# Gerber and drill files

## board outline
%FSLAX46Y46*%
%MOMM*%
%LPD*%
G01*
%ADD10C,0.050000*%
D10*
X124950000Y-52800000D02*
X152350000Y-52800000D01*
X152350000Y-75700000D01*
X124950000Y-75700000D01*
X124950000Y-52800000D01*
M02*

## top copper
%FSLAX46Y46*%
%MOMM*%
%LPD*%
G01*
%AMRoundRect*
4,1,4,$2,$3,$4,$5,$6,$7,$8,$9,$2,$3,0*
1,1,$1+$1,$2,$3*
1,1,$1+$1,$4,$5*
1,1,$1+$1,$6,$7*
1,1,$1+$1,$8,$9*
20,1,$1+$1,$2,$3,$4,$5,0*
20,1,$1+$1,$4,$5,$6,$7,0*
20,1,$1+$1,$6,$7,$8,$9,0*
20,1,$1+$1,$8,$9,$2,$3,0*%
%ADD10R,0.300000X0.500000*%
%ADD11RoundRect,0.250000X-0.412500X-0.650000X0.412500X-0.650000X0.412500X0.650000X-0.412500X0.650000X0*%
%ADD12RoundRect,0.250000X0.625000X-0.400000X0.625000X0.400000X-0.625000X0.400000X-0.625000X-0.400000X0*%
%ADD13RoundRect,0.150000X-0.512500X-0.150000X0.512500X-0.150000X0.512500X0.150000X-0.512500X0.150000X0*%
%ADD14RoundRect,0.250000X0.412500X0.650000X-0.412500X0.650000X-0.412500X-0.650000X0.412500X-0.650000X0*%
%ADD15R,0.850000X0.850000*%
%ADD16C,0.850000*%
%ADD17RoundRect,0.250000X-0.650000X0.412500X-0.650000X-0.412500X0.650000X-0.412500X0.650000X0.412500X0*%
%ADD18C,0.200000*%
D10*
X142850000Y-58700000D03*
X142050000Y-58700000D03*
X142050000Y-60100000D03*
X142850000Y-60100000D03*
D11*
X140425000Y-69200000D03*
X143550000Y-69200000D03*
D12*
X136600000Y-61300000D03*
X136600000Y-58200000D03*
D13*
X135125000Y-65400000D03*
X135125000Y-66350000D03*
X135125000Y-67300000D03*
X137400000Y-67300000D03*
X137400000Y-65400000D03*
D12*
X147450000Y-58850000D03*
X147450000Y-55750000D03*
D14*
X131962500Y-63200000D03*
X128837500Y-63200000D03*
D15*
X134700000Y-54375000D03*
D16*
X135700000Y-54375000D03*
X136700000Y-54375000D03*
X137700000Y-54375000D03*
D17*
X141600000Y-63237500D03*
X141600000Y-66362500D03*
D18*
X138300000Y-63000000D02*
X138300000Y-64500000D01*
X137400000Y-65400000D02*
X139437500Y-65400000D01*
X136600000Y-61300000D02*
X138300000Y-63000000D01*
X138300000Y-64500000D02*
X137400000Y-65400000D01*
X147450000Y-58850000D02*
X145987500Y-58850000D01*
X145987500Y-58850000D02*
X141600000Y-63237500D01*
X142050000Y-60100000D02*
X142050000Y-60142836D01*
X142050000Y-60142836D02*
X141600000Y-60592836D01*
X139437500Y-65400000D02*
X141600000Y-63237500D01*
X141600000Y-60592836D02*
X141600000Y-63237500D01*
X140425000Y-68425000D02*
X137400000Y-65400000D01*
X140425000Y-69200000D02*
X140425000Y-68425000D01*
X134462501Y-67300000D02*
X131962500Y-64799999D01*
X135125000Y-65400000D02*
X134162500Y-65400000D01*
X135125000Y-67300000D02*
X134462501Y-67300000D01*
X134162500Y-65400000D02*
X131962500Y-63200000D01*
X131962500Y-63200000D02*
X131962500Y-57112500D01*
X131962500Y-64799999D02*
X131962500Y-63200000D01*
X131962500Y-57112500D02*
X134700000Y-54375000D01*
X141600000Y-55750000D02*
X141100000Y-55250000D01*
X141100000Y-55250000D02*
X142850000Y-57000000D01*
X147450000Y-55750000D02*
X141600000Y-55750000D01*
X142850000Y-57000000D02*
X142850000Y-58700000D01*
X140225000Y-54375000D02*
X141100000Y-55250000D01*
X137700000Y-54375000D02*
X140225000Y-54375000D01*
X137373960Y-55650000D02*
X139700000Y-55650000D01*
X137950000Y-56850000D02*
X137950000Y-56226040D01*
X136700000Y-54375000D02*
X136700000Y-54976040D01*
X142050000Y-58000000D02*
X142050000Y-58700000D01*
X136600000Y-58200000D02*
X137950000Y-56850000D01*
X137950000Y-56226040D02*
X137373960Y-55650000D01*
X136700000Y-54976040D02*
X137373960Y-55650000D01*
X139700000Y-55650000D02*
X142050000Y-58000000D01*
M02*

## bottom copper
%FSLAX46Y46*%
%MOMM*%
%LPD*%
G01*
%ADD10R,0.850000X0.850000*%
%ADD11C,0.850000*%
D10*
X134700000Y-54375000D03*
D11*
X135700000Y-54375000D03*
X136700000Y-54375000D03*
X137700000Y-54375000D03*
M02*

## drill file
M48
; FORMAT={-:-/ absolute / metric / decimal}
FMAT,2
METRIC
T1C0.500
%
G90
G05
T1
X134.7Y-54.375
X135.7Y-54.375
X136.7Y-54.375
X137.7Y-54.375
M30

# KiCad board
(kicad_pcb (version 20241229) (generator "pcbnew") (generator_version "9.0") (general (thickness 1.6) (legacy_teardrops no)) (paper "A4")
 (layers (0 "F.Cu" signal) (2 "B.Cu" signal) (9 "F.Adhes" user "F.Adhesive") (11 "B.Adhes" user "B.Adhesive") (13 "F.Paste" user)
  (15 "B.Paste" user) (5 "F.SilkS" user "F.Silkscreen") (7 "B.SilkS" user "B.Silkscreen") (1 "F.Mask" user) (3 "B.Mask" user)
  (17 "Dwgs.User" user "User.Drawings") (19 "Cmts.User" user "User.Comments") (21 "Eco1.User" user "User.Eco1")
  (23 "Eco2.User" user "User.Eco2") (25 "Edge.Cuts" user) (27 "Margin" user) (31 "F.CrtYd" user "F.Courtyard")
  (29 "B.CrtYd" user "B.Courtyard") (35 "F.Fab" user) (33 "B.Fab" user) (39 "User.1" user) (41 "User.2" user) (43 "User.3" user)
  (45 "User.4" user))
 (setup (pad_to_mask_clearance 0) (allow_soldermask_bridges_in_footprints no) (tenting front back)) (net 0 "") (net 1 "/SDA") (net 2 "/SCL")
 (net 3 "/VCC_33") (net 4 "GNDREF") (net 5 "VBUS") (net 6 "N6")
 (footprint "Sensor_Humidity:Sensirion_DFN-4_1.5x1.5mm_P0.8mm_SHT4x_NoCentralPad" (layer "F.Cu") (at 142.45 59.4 -90)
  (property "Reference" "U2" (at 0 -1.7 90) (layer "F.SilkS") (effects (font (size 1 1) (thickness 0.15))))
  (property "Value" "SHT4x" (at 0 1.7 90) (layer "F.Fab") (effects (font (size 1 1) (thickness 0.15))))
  (pad "1" smd rect (at -0.7 -0.4 270) (size 0.5 0.3) (layers "F.Cu" "F.Mask" "F.Paste") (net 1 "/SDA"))
  (pad "2" smd rect (at -0.7 0.4 270) (size 0.5 0.3) (layers "F.Cu" "F.Mask" "F.Paste") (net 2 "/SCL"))
  (pad "3" smd rect (at 0.7 0.4 270) (size 0.5 0.3) (layers "F.Cu" "F.Mask" "F.Paste") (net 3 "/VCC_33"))
  (pad "4" smd rect (at 0.7 -0.4 270) (size 0.5 0.3) (layers "F.Cu" "F.Mask" "F.Paste") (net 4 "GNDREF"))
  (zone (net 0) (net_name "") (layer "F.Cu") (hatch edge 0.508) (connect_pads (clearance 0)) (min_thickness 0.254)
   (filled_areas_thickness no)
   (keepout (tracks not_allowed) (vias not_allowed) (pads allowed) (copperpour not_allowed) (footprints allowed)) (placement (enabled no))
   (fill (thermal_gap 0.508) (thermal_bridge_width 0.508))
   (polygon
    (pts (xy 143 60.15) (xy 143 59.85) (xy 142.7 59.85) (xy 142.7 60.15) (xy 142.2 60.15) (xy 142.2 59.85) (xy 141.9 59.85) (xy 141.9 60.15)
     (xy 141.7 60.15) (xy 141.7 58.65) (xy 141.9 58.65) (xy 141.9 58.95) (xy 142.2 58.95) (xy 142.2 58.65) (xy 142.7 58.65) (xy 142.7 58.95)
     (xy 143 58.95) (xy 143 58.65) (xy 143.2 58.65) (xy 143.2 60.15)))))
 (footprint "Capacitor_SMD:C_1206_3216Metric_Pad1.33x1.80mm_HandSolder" (layer "F.Cu") (at 141.9875 69.2)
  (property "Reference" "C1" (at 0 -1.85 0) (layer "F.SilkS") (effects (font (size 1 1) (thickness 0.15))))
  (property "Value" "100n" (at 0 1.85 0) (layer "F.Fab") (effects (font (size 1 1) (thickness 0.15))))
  (pad "1" smd roundrect (at -1.5625 0) (size 1.325 1.8) (layers "F.Cu" "F.Mask" "F.Paste") (roundrect_rratio 0.188679) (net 3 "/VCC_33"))
  (pad "2" smd roundrect (at 1.5625 0) (size 1.325 1.8) (layers "F.Cu" "F.Mask" "F.Paste") (roundrect_rratio 0.188679) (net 4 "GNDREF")))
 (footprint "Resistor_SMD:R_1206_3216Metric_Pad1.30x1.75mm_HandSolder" (layer "F.Cu") (at 136.6 59.75 90)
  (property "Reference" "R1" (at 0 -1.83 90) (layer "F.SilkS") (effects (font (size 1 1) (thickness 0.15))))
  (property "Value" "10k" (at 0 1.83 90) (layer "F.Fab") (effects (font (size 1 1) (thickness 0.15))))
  (pad "1" smd roundrect (at -1.55 0 90) (size 1.3 1.75) (layers "F.Cu" "F.Mask" "F.Paste") (roundrect_rratio 0.192308) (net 3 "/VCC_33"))
  (pad "2" smd roundrect (at 1.55 0 90) (size 1.3 1.75) (layers "F.Cu" "F.Mask" "F.Paste") (roundrect_rratio 0.192308) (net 2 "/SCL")))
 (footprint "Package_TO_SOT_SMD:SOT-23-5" (layer "F.Cu") (at 136.2625 66.35)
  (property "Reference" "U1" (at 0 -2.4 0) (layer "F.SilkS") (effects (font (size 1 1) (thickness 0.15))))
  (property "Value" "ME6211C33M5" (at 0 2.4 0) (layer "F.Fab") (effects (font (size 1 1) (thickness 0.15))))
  (pad "1" smd roundrect (at -1.1375 -0.95) (size 1.325 0.6) (layers "F.Cu" "F.Mask" "F.Paste") (roundrect_rratio 0.25) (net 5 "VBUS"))
  (pad "2" smd roundrect (at -1.1375 0) (size 1.325 0.6) (layers "F.Cu" "F.Mask" "F.Paste") (roundrect_rratio 0.25) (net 4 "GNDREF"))
  (pad "3" smd roundrect (at -1.1375 0.95) (size 1.325 0.6) (layers "F.Cu" "F.Mask" "F.Paste") (roundrect_rratio 0.25) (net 5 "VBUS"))
  (pad "4" smd roundrect (at 1.1375 0.95) (size 1.325 0.6) (layers "F.Cu" "F.Mask" "F.Paste") (roundrect_rratio 0.25) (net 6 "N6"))
  (pad "5" smd roundrect (at 1.1375 -0.95) (size 1.325 0.6) (layers "F.Cu" "F.Mask" "F.Paste") (roundrect_rratio 0.25) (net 3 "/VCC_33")))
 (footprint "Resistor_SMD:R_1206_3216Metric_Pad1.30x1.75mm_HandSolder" (layer "F.Cu") (at 147.45 57.3 90)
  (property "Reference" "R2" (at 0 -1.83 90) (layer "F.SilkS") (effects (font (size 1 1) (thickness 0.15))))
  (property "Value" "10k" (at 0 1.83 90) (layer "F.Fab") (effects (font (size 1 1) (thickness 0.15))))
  (pad "1" smd roundrect (at -1.55 0 90) (size 1.3 1.75) (layers "F.Cu" "F.Mask" "F.Paste") (roundrect_rratio 0.192308) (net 3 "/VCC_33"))
  (pad "2" smd roundrect (at 1.55 0 90) (size 1.3 1.75) (layers "F.Cu" "F.Mask" "F.Paste") (roundrect_rratio 0.192308) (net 1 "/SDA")))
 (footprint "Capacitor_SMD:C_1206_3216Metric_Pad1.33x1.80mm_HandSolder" (layer "F.Cu") (at 130.4 63.2 180)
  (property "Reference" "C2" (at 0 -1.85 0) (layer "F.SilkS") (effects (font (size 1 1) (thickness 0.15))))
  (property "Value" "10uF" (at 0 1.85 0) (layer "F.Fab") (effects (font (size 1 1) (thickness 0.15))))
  (pad "1" smd roundrect (at -1.5625 0 180) (size 1.325 1.8) (layers "F.Cu" "F.Mask" "F.Paste") (roundrect_rratio 0.188679) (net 5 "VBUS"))
  (pad "2" smd roundrect (at 1.5625 0 180) (size 1.325 1.8) (layers "F.Cu" "F.Mask" "F.Paste") (roundrect_rratio 0.188679) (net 4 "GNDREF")))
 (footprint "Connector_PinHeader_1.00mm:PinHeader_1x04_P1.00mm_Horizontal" (layer "F.Cu") (at 134.7 54.375 90)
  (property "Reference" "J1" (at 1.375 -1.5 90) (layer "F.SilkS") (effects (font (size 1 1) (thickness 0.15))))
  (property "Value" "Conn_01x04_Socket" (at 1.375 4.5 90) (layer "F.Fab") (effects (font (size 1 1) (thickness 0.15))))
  (pad "1" thru_hole rect (at 0 0 90) (size 0.85 0.85) (drill 0.5) (layers "*.Cu" "*.Mask") (remove_unused_layers no) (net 5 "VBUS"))
  (pad "2" thru_hole circle (at 0 1 90) (size 0.85 0.85) (drill 0.5) (layers "*.Cu" "*.Mask") (remove_unused_layers no) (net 4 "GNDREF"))
  (pad "3" thru_hole circle (at 0 2 90) (size 0.85 0.85) (drill 0.5) (layers "*.Cu" "*.Mask") (remove_unused_layers no) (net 2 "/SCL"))
  (pad "4" thru_hole circle (at 0 3 90) (size 0.85 0.85) (drill 0.5) (layers "*.Cu" "*.Mask") (remove_unused_layers no) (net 1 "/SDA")))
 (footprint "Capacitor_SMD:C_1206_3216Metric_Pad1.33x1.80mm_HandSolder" (layer "F.Cu") (at 141.6 64.8 -90)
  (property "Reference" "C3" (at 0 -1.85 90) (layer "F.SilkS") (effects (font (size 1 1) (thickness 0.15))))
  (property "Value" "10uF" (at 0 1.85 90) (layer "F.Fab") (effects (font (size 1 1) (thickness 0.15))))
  (pad "1" smd roundrect (at -1.5625 0 270) (size 1.325 1.8) (layers "F.Cu" "F.Mask" "F.Paste") (roundrect_rratio 0.188679)
   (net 3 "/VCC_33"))
  (pad "2" smd roundrect (at 1.5625 0 270) (size 1.325 1.8) (layers "F.Cu" "F.Mask" "F.Paste") (roundrect_rratio 0.188679) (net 4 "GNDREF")))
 (gr_rect (start 124.95 52.8) (end 152.35 75.7) (stroke (width 0.05) (type default)) (fill no) (layer "Edge.Cuts"))
 (segment (start 138.3 63) (end 138.3 64.5) (width 0.2) (layer "F.Cu") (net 3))
 (segment (start 137.4 65.4) (end 139.4375 65.4) (width 0.2) (layer "F.Cu") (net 3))
 (segment (start 136.6 61.3) (end 138.3 63) (width 0.2) (layer "F.Cu") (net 3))
 (segment (start 138.3 64.5) (end 137.4 65.4) (width 0.2) (layer "F.Cu") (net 3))
 (segment (start 147.45 58.85) (end 145.9875 58.85) (width 0.2) (layer "F.Cu") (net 3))
 (segment (start 145.9875 58.85) (end 141.6 63.2375) (width 0.2) (layer "F.Cu") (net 3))
 (segment (start 142.05 60.1) (end 142.05 60.142836) (width 0.2) (layer "F.Cu") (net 3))
 (segment (start 142.05 60.142836) (end 141.6 60.592836) (width 0.2) (layer "F.Cu") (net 3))
 (segment (start 139.4375 65.4) (end 141.6 63.2375) (width 0.2) (layer "F.Cu") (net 3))
 (segment (start 141.6 60.592836) (end 141.6 63.2375) (width 0.2) (layer "F.Cu") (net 3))
 (segment (start 140.425 68.425) (end 137.4 65.4) (width 0.2) (layer "F.Cu") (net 3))
 (segment (start 140.425 69.2) (end 140.425 68.425) (width 0.2) (layer "F.Cu") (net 3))
 (segment (start 134.462501 67.3) (end 131.9625 64.799999) (width 0.2) (layer "F.Cu") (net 5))
 (segment (start 135.125 65.4) (end 134.1625 65.4) (width 0.2) (layer "F.Cu") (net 5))
 (segment (start 135.125 67.3) (end 134.462501 67.3) (width 0.2) (layer "F.Cu") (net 5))
 (segment (start 134.1625 65.4) (end 131.9625 63.2) (width 0.2) (layer "F.Cu") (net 5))
 (segment (start 131.9625 63.2) (end 131.9625 57.1125) (width 0.2) (layer "F.Cu") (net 5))
 (segment (start 131.9625 64.799999) (end 131.9625 63.2) (width 0.2) (layer "F.Cu") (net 5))
 (segment (start 131.9625 57.1125) (end 134.7 54.375) (width 0.2) (layer "F.Cu") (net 5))
 (segment (start 141.6 55.75) (end 141.1 55.25) (width 0.2) (layer "F.Cu") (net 1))
 (segment (start 141.1 55.25) (end 142.85 57) (width 0.2) (layer "F.Cu") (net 1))
 (segment (start 147.45 55.75) (end 141.6 55.75) (width 0.2) (layer "F.Cu") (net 1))
 (segment (start 142.85 57) (end 142.85 58.7) (width 0.2) (layer "F.Cu") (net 1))
 (segment (start 140.225 54.375) (end 141.1 55.25) (width 0.2) (layer "F.Cu") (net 1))
 (segment (start 137.7 54.375) (end 140.225 54.375) (width 0.2) (layer "F.Cu") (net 1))
 (segment (start 137.37396 55.65) (end 139.7 55.65) (width 0.2) (layer "F.Cu") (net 2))
 (segment (start 137.95 56.85) (end 137.95 56.22604) (width 0.2) (layer "F.Cu") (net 2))
 (segment (start 136.7 54.375) (end 136.7 54.97604) (width 0.2) (layer "F.Cu") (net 2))
 (segment (start 142.05 58) (end 142.05 58.7) (width 0.2) (layer "F.Cu") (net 2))
 (segment (start 136.6 58.2) (end 137.95 56.85) (width 0.2) (layer "F.Cu") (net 2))
 (segment (start 137.95 56.22604) (end 137.37396 55.65) (width 0.2) (layer "F.Cu") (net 2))
 (segment (start 136.7 54.97604) (end 137.37396 55.65) (width 0.2) (layer "F.Cu") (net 2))
 (segment (start 139.7 55.65) (end 142.05 58) (width 0.2) (layer "F.Cu") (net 2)))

